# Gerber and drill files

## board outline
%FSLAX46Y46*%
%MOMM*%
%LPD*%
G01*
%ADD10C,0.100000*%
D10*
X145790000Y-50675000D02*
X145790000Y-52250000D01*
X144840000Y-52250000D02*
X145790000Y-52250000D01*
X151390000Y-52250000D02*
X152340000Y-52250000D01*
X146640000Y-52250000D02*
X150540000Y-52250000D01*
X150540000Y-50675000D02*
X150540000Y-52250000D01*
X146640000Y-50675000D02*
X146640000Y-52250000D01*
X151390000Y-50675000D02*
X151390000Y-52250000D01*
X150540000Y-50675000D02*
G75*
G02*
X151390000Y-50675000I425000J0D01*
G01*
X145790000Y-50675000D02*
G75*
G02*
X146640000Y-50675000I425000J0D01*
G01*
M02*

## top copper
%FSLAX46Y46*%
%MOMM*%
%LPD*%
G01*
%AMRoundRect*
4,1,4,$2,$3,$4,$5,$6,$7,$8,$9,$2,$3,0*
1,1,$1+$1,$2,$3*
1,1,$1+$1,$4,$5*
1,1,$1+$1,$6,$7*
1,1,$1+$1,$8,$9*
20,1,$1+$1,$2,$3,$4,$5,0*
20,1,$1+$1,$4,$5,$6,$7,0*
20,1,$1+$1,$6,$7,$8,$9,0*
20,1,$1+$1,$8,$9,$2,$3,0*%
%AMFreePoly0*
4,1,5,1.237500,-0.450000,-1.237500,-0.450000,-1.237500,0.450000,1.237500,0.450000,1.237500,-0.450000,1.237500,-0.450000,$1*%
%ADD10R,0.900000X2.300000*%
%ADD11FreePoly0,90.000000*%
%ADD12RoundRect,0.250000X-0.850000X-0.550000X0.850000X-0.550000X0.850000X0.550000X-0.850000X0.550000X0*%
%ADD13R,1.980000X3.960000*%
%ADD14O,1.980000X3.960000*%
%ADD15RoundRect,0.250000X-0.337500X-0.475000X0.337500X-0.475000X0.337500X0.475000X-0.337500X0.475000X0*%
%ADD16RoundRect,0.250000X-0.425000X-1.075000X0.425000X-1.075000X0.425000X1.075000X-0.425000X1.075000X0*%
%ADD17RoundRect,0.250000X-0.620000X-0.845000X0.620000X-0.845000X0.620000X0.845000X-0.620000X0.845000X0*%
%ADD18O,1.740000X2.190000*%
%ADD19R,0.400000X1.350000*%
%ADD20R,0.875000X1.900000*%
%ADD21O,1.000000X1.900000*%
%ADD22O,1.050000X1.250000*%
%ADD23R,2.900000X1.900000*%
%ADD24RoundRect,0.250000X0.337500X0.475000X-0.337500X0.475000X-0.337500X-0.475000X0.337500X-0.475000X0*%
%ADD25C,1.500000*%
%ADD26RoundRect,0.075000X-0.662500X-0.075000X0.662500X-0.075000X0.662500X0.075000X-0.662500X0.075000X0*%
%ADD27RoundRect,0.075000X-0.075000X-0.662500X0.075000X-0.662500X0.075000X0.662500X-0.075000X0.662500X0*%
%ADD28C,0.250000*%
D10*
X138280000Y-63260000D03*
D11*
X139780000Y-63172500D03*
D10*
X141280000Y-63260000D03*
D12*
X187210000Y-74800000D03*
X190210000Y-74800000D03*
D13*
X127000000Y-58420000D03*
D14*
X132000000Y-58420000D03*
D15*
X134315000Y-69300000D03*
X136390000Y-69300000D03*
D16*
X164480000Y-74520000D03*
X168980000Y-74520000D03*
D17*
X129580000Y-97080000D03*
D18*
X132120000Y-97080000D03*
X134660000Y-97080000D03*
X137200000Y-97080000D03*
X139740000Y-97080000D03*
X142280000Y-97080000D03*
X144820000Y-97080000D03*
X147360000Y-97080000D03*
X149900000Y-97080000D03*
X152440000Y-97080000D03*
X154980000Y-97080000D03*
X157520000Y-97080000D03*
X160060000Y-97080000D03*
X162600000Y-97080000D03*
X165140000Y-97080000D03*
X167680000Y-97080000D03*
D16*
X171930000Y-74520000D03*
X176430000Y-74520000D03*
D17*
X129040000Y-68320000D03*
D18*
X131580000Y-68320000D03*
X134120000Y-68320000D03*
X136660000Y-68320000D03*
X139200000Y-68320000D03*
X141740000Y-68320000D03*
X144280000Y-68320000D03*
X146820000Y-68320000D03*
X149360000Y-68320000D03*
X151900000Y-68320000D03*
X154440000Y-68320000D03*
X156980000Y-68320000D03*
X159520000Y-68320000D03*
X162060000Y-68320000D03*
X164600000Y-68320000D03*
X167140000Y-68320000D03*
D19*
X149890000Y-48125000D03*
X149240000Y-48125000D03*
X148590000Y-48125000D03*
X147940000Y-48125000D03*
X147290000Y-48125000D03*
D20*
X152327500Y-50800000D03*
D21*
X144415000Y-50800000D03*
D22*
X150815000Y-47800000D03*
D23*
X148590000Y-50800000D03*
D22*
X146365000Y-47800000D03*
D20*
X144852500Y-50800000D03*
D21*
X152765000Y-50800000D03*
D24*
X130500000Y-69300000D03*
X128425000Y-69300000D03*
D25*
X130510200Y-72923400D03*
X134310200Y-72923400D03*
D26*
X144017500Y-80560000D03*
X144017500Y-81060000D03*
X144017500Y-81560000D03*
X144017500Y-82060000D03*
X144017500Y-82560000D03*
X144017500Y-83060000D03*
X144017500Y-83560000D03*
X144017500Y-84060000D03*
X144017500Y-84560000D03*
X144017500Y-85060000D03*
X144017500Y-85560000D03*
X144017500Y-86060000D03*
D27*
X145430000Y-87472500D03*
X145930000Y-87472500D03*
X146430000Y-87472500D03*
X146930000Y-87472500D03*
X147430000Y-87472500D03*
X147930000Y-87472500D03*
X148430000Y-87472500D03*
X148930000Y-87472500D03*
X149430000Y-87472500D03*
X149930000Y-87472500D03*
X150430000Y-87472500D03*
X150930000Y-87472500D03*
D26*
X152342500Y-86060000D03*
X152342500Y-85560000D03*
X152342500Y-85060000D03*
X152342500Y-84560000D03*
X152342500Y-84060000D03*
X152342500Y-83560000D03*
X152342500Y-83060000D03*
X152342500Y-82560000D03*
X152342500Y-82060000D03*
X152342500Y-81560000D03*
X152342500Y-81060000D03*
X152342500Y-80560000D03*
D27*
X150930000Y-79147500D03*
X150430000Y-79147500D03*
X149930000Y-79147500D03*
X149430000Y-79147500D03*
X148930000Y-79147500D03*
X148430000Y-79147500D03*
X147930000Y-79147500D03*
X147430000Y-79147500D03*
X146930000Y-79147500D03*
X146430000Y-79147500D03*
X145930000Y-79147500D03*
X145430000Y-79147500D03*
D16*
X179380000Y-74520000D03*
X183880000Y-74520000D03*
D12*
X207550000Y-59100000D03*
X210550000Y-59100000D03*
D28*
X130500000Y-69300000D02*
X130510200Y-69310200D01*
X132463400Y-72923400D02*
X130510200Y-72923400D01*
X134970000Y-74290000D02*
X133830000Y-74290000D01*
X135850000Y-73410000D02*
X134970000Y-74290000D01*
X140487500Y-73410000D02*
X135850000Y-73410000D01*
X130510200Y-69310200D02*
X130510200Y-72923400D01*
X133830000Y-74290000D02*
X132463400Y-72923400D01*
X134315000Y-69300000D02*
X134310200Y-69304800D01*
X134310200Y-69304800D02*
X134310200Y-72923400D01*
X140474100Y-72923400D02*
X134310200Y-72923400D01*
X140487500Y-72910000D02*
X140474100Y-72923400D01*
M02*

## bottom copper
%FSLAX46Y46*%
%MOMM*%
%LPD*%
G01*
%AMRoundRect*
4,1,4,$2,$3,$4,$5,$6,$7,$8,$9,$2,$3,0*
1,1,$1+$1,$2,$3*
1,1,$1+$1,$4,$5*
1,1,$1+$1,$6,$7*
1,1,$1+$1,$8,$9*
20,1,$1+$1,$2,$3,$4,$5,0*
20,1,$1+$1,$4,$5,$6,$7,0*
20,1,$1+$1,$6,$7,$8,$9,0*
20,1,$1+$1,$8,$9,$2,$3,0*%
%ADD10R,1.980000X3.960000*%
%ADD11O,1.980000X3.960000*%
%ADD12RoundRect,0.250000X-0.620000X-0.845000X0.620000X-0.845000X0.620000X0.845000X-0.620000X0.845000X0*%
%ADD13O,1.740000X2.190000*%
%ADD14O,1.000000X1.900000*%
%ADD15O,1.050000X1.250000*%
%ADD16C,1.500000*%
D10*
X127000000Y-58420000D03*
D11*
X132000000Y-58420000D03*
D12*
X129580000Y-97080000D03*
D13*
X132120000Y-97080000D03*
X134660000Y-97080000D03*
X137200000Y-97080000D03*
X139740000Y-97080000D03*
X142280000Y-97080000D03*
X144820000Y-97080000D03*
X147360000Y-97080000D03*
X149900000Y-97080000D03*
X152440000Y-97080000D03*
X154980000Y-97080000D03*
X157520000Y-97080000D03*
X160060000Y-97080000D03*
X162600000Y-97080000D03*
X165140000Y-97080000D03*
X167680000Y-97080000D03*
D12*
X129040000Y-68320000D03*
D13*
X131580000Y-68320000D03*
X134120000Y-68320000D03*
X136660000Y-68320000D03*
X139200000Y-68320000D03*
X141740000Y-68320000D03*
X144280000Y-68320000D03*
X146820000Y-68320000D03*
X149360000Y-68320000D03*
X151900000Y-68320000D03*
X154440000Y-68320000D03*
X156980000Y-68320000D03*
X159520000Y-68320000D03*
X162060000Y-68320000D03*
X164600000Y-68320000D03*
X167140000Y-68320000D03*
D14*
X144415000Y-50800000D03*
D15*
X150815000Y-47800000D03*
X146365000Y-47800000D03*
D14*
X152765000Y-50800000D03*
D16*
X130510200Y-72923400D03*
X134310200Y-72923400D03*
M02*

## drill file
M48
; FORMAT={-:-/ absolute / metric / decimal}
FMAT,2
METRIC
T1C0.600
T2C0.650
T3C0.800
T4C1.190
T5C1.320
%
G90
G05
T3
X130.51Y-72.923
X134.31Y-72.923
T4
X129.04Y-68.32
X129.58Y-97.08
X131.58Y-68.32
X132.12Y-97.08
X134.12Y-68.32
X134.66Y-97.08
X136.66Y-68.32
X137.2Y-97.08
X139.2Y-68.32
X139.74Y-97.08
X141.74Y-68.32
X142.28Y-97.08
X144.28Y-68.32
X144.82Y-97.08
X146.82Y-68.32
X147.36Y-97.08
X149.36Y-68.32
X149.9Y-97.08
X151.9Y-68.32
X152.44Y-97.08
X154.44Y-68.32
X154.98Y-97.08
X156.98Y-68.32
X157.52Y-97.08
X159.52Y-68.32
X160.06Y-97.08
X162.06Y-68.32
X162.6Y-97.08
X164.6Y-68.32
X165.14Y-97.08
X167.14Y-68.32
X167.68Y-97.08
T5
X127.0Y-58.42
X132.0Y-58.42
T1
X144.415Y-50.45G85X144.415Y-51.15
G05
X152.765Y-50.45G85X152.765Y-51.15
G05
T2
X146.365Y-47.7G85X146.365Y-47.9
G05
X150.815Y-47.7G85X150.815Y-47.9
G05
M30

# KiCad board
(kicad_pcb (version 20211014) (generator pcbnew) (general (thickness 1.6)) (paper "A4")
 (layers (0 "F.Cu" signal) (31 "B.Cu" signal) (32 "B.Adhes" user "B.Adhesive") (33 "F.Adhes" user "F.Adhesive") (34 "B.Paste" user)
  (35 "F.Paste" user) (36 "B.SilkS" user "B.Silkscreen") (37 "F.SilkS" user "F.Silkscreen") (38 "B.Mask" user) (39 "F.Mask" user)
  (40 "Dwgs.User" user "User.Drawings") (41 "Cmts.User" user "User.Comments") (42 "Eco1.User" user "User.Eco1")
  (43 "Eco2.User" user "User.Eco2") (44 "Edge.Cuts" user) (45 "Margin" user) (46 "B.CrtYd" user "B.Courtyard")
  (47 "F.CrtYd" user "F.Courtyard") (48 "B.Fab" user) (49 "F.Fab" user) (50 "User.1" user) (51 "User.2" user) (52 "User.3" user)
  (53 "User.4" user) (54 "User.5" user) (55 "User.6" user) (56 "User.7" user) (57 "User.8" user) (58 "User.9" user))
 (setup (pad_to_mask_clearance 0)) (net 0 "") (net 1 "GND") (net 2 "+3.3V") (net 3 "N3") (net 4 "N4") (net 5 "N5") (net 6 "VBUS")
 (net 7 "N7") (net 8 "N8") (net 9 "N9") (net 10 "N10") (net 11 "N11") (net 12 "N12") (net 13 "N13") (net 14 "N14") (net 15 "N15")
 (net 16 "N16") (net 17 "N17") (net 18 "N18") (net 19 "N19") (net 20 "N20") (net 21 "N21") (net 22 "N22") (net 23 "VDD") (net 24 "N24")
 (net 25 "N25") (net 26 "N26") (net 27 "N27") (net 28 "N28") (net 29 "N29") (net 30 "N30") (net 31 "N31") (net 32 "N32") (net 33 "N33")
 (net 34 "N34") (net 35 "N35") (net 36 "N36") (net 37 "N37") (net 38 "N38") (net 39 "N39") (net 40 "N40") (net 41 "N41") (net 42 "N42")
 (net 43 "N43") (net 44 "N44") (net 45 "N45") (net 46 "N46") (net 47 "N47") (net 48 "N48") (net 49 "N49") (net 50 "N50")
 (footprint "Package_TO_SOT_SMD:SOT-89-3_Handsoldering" (layer "F.Cu") (at 139.78 61.11 90)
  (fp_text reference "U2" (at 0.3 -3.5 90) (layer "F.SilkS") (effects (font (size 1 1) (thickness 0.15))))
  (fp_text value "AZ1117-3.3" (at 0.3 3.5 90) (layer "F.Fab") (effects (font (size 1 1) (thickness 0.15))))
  (pad "1" smd rect (at -2.15 -1.5 90) (size 2.3 0.9) (layers "F.Cu" "F.Paste" "F.Mask") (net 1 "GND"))
  (pad "2" smd custom (at -2.0625 0 90) (size 2.475 0.9) (layers "F.Cu" "F.Paste" "F.Mask") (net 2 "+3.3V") (zone_connect 2)
   (options (clearance outline) (anchor rect)) (primitives))
  (pad "3" smd rect (at -2.15 1.5 90) (size 2.3 0.9) (layers "F.Cu" "F.Paste" "F.Mask") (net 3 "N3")))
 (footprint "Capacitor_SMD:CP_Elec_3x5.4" (layer "F.Cu") (at 188.71 74.8)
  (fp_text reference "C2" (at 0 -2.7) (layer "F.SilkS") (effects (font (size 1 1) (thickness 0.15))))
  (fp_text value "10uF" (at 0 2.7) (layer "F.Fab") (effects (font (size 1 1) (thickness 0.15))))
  (pad "1" smd roundrect (at -1.5 0) (size 2.2 1.6) (layers "F.Cu" "F.Paste" "F.Mask") (roundrect_rratio 0.15625) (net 2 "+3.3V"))
  (pad "2" smd roundrect (at 1.5 0) (size 2.2 1.6) (layers "F.Cu" "F.Paste" "F.Mask") (roundrect_rratio 0.15625) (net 1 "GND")))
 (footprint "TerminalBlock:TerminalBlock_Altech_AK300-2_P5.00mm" (layer "F.Cu") (at 127 58.42)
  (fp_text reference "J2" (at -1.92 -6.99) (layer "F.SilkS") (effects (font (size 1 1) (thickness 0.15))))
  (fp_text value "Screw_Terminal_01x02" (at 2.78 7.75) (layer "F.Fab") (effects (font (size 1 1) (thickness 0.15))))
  (pad "1" thru_hole rect (at 0 0) (size 1.98 3.96) (drill 1.32) (layers *.Cu *.Mask) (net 1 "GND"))
  (pad "2" thru_hole oval (at 5 0) (size 1.98 3.96) (drill 1.32) (layers *.Cu *.Mask) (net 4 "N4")))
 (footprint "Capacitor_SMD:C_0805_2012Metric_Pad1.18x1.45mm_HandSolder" (layer "F.Cu") (at 135.3525 69.3)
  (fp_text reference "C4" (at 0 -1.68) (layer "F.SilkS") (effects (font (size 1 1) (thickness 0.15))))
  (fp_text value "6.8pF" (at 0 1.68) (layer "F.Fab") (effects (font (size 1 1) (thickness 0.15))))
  (pad "1" smd roundrect (at -1.0375 0) (size 1.175 1.45) (layers "F.Cu" "F.Paste" "F.Mask") (roundrect_rratio 0.212766) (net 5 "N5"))
  (pad "2" smd roundrect (at 1.0375 0) (size 1.175 1.45) (layers "F.Cu" "F.Paste" "F.Mask") (roundrect_rratio 0.212766) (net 1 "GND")))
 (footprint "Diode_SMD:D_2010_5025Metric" (layer "F.Cu") (at 166.73 74.52)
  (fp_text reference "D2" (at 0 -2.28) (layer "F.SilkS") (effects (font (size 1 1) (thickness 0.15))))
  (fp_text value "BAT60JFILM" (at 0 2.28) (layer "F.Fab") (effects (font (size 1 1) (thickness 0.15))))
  (pad "1" smd roundrect (at -2.25 0) (size 1.35 2.65) (layers "F.Cu" "F.Paste" "F.Mask") (roundrect_rratio 0.185185) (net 3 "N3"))
  (pad "2" smd roundrect (at 2.25 0) (size 1.35 2.65) (layers "F.Cu" "F.Paste" "F.Mask") (roundrect_rratio 0.185185) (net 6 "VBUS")))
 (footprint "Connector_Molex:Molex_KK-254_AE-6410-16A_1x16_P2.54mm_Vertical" (layer "F.Cu") (at 129.58 97.08)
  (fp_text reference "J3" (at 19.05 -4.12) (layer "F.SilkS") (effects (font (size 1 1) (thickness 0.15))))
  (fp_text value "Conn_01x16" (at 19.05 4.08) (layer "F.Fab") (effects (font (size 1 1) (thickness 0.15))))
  (pad "1" thru_hole roundrect (at 0 0) (size 1.74 2.19) (drill 1.19) (layers *.Cu *.Mask) (roundrect_rratio 0.143678) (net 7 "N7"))
  (pad "2" thru_hole oval (at 2.54 0) (size 1.74 2.19) (drill 1.19) (layers *.Cu *.Mask) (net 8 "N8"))
  (pad "3" thru_hole oval (at 5.08 0) (size 1.74 2.19) (drill 1.19) (layers *.Cu *.Mask) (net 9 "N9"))
  (pad "4" thru_hole oval (at 7.62 0) (size 1.74 2.19) (drill 1.19) (layers *.Cu *.Mask) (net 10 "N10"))
  (pad "5" thru_hole oval (at 10.16 0) (size 1.74 2.19) (drill 1.19) (layers *.Cu *.Mask) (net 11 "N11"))
  (pad "6" thru_hole oval (at 12.7 0) (size 1.74 2.19) (drill 1.19) (layers *.Cu *.Mask) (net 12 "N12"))
  (pad "7" thru_hole oval (at 15.24 0) (size 1.74 2.19) (drill 1.19) (layers *.Cu *.Mask) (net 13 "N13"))
  (pad "8" thru_hole oval (at 17.78 0) (size 1.74 2.19) (drill 1.19) (layers *.Cu *.Mask) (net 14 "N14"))
  (pad "9" thru_hole oval (at 20.32 0) (size 1.74 2.19) (drill 1.19) (layers *.Cu *.Mask) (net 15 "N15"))
  (pad "10" thru_hole oval (at 22.86 0) (size 1.74 2.19) (drill 1.19) (layers *.Cu *.Mask) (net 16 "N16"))
  (pad "11" thru_hole oval (at 25.4 0) (size 1.74 2.19) (drill 1.19) (layers *.Cu *.Mask) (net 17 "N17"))
  (pad "12" thru_hole oval (at 27.94 0) (size 1.74 2.19) (drill 1.19) (layers *.Cu *.Mask) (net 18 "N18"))
  (pad "13" thru_hole oval (at 30.48 0) (size 1.74 2.19) (drill 1.19) (layers *.Cu *.Mask) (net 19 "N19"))
  (pad "14" thru_hole oval (at 33.02 0) (size 1.74 2.19) (drill 1.19) (layers *.Cu *.Mask) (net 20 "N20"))
  (pad "15" thru_hole oval (at 35.56 0) (size 1.74 2.19) (drill 1.19) (layers *.Cu *.Mask) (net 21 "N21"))
  (pad "16" thru_hole oval (at 38.1 0) (size 1.74 2.19) (drill 1.19) (layers *.Cu *.Mask) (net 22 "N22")))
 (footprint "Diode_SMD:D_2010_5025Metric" (layer "F.Cu") (at 174.18 74.52)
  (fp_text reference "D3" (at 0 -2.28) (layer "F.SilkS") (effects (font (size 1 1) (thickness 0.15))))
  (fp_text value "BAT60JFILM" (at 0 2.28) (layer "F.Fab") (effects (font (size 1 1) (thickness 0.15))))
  (pad "1" smd roundrect (at -2.25 0) (size 1.35 2.65) (layers "F.Cu" "F.Paste" "F.Mask") (roundrect_rratio 0.185185) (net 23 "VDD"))
  (pad "2" smd roundrect (at 2.25 0) (size 1.35 2.65) (layers "F.Cu" "F.Paste" "F.Mask") (roundrect_rratio 0.185185) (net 2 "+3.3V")))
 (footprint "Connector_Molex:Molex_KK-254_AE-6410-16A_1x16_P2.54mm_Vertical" (layer "F.Cu") (at 129.04 68.32)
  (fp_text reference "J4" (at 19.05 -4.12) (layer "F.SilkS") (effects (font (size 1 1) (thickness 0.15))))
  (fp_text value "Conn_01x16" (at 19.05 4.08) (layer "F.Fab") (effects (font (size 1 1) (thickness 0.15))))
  (pad "1" thru_hole roundrect (at 0 0) (size 1.74 2.19) (drill 1.19) (layers *.Cu *.Mask) (roundrect_rratio 0.143678) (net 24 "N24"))
  (pad "2" thru_hole oval (at 2.54 0) (size 1.74 2.19) (drill 1.19) (layers *.Cu *.Mask) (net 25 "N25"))
  (pad "3" thru_hole oval (at 5.08 0) (size 1.74 2.19) (drill 1.19) (layers *.Cu *.Mask) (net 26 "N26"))
  (pad "4" thru_hole oval (at 7.62 0) (size 1.74 2.19) (drill 1.19) (layers *.Cu *.Mask) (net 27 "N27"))
  (pad "5" thru_hole oval (at 10.16 0) (size 1.74 2.19) (drill 1.19) (layers *.Cu *.Mask) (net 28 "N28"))
  (pad "6" thru_hole oval (at 12.7 0) (size 1.74 2.19) (drill 1.19) (layers *.Cu *.Mask) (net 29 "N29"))
  (pad "7" thru_hole oval (at 15.24 0) (size 1.74 2.19) (drill 1.19) (layers *.Cu *.Mask) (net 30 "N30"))
  (pad "8" thru_hole oval (at 17.78 0) (size 1.74 2.19) (drill 1.19) (layers *.Cu *.Mask) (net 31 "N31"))
  (pad "9" thru_hole oval (at 20.32 0) (size 1.74 2.19) (drill 1.19) (layers *.Cu *.Mask) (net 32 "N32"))
  (pad "10" thru_hole oval (at 22.86 0) (size 1.74 2.19) (drill 1.19) (layers *.Cu *.Mask) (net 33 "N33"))
  (pad "11" thru_hole oval (at 25.4 0) (size 1.74 2.19) (drill 1.19) (layers *.Cu *.Mask) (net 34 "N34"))
  (pad "12" thru_hole oval (at 27.94 0) (size 1.74 2.19) (drill 1.19) (layers *.Cu *.Mask) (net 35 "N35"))
  (pad "13" thru_hole oval (at 30.48 0) (size 1.74 2.19) (drill 1.19) (layers *.Cu *.Mask) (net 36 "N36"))
  (pad "14" thru_hole oval (at 33.02 0) (size 1.74 2.19) (drill 1.19) (layers *.Cu *.Mask) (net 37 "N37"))
  (pad "15" thru_hole oval (at 35.56 0) (size 1.74 2.19) (drill 1.19) (layers *.Cu *.Mask) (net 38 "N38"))
  (pad "16" thru_hole oval (at 38.1 0) (size 1.74 2.19) (drill 1.19) (layers *.Cu *.Mask) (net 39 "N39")))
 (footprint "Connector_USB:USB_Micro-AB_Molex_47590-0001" (layer "F.Cu") (at 148.59 50.8)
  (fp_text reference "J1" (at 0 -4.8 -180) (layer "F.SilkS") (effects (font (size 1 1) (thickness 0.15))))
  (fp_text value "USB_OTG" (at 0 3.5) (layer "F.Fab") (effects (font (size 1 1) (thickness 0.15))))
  (fp_line (start -2.8 -0.125) (end -2.8 1.45) (layer "Edge.Cuts") (width 0.1))
  (fp_line (start -3.75 1.45) (end -2.8 1.45) (layer "Edge.Cuts") (width 0.1))
  (fp_line (start 2.8 1.45) (end 3.75 1.45) (layer "Edge.Cuts") (width 0.1))
  (fp_line (start -1.95 1.45) (end 1.95 1.45) (layer "Edge.Cuts") (width 0.1))
  (fp_line (start 1.95 -0.125) (end 1.95 1.45) (layer "Edge.Cuts") (width 0.1))
  (fp_line (start -1.95 -0.125) (end -1.95 1.45) (layer "Edge.Cuts") (width 0.1))
  (fp_line (start 2.8 -0.125) (end 2.8 1.45) (layer "Edge.Cuts") (width 0.1))
  (fp_arc (start 1.95 -0.125) (mid 2.375 -0.55) (end 2.8 -0.125) (layer "Edge.Cuts") (width 0.1))
  (fp_arc (start -2.8 -0.125) (mid -2.375 -0.55) (end -1.95 -0.125) (layer "Edge.Cuts") (width 0.1))
  (pad "" smd rect (at 3.5 0) (size 0.3 0.85) (layers "F.Paste"))
  (pad "" smd rect (at -3.5 0) (size 0.3 0.85) (layers "F.Paste"))
  (pad "1" smd rect (at 1.3 -2.675) (size 0.4 1.35) (layers "F.Cu" "F.Paste" "F.Mask") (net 6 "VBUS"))
  (pad "2" smd rect (at 0.65 -2.675) (size 0.4 1.35) (layers "F.Cu" "F.Paste" "F.Mask") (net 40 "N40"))
  (pad "3" smd rect (at 0 -2.675) (size 0.4 1.35) (layers "F.Cu" "F.Paste" "F.Mask") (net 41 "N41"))
  (pad "4" smd rect (at -0.65 -2.675) (size 0.4 1.35) (layers "F.Cu" "F.Paste" "F.Mask") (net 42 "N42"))
  (pad "5" smd rect (at -1.3 -2.675) (size 0.4 1.35) (layers "F.Cu" "F.Paste" "F.Mask") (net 1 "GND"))
  (pad "6" smd rect (at 3.7375 0) (size 0.875 1.9) (layers "F.Cu" "F.Mask") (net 1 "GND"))
  (pad "6" thru_hole oval (at -4.175 0) (size 1 1.9) (drill oval 0.6 1.3) (layers *.Cu *.Mask) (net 1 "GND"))
  (pad "6" thru_hole oval (at 2.225 -3) (size 1.05 1.25) (drill oval 0.65 0.85) (layers *.Cu *.Mask) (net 1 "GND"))
  (pad "6" smd rect (at 0 0) (size 2.9 1.9) (layers "F.Cu" "F.Paste" "F.Mask") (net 1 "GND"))
  (pad "6" thru_hole oval (at -2.225 -3) (size 1.05 1.25) (drill oval 0.65 0.85) (layers *.Cu *.Mask) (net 1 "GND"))
  (pad "6" smd rect (at -3.7375 0) (size 0.875 1.9) (layers "F.Cu" "F.Mask") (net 1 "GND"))
  (pad "6" thru_hole oval (at 4.175 0) (size 1 1.9) (drill oval 0.6 1.3) (layers *.Cu *.Mask) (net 1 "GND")))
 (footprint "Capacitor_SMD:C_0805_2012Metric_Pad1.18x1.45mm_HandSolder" (layer "F.Cu") (at 129.4625 69.3 180)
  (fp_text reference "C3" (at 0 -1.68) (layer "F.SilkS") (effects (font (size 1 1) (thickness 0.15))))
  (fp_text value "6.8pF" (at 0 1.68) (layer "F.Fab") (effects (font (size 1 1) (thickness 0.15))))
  (pad "1" smd roundrect (at -1.0375 0 180) (size 1.175 1.45) (layers "F.Cu" "F.Paste" "F.Mask") (roundrect_rratio 0.212766) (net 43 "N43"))
  (pad "2" smd roundrect (at 1.0375 0 180) (size 1.175 1.45) (layers "F.Cu" "F.Paste" "F.Mask") (roundrect_rratio 0.212766) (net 1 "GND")))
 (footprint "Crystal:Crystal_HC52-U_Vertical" (layer "F.Cu") (at 130.5102 72.9234)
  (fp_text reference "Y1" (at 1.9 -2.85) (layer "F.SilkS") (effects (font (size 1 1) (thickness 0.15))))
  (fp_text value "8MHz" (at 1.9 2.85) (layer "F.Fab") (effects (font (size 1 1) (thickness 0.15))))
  (pad "1" thru_hole circle (at 0 0) (size 1.5 1.5) (drill 0.8) (layers *.Cu *.Mask) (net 43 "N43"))
  (pad "2" thru_hole circle (at 3.8 0) (size 1.5 1.5) (drill 0.8) (layers *.Cu *.Mask) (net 5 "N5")))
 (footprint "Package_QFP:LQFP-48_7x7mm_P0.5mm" (layer "F.Cu") (at 148.18 83.31)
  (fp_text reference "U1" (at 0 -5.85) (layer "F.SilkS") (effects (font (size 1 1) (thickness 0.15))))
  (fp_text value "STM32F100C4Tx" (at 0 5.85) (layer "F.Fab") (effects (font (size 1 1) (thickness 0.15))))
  (pad "1" smd roundrect (at -4.1625 -2.75) (size 1.475 0.3) (layers "F.Cu" "F.Paste" "F.Mask") (roundrect_rratio 0.25) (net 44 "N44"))
  (pad "2" smd roundrect (at -4.1625 -2.25) (size 1.475 0.3) (layers "F.Cu" "F.Paste" "F.Mask") (roundrect_rratio 0.25) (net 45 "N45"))
  (pad "3" smd roundrect (at -4.1625 -1.75) (size 1.475 0.3) (layers "F.Cu" "F.Paste" "F.Mask") (roundrect_rratio 0.25) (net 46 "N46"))
  (pad "4" smd roundrect (at -4.1625 -1.25) (size 1.475 0.3) (layers "F.Cu" "F.Paste" "F.Mask") (roundrect_rratio 0.25) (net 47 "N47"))
  (pad "5" smd roundrect (at -4.1625 -0.75) (size 1.475 0.3) (layers "F.Cu" "F.Paste" "F.Mask") (roundrect_rratio 0.25) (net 5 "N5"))
  (pad "6" smd roundrect (at -4.1625 -0.25) (size 1.475 0.3) (layers "F.Cu" "F.Paste" "F.Mask") (roundrect_rratio 0.25) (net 43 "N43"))
  (pad "7" smd roundrect (at -4.1625 0.25) (size 1.475 0.3) (layers "F.Cu" "F.Paste" "F.Mask") (roundrect_rratio 0.25) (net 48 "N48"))
  (pad "8" smd roundrect (at -4.1625 0.75) (size 1.475 0.3) (layers "F.Cu" "F.Paste" "F.Mask") (roundrect_rratio 0.25) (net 1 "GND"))
  (pad "9" smd roundrect (at -4.1625 1.25) (size 1.475 0.3) (layers "F.Cu" "F.Paste" "F.Mask") (roundrect_rratio 0.25) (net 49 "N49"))
  (pad "10" smd roundrect (at -4.1625 1.75) (size 1.475 0.3) (layers "F.Cu" "F.Paste" "F.Mask") (roundrect_rratio 0.25) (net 7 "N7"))
  (pad "11" smd roundrect (at -4.1625 2.25) (size 1.475 0.3) (layers "F.Cu" "F.Paste" "F.Mask") (roundrect_rratio 0.25) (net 8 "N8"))
  (pad "12" smd roundrect (at -4.1625 2.75) (size 1.475 0.3) (layers "F.Cu" "F.Paste" "F.Mask") (roundrect_rratio 0.25) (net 9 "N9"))
  (pad "13" smd roundrect (at -2.75 4.1625) (size 0.3 1.475) (layers "F.Cu" "F.Paste" "F.Mask") (roundrect_rratio 0.25) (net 10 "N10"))
  (pad "14" smd roundrect (at -2.25 4.1625) (size 0.3 1.475) (layers "F.Cu" "F.Paste" "F.Mask") (roundrect_rratio 0.25) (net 11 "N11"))
  (pad "15" smd roundrect (at -1.75 4.1625) (size 0.3 1.475) (layers "F.Cu" "F.Paste" "F.Mask") (roundrect_rratio 0.25) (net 12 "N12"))
  (pad "16" smd roundrect (at -1.25 4.1625) (size 0.3 1.475) (layers "F.Cu" "F.Paste" "F.Mask") (roundrect_rratio 0.25) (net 13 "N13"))
  (pad "17" smd roundrect (at -0.75 4.1625) (size 0.3 1.475) (layers "F.Cu" "F.Paste" "F.Mask") (roundrect_rratio 0.25) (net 14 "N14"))
  (pad "18" smd roundrect (at -0.25 4.1625) (size 0.3 1.475) (layers "F.Cu" "F.Paste" "F.Mask") (roundrect_rratio 0.25) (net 24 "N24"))
  (pad "19" smd roundrect (at 0.25 4.1625) (size 0.3 1.475) (layers "F.Cu" "F.Paste" "F.Mask") (roundrect_rratio 0.25) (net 25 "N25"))
  (pad "20" smd roundrect (at 0.75 4.1625) (size 0.3 1.475) (layers "F.Cu" "F.Paste" "F.Mask") (roundrect_rratio 0.25) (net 26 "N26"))
  (pad "21" smd roundrect (at 1.25 4.1625) (size 0.3 1.475) (layers "F.Cu" "F.Paste" "F.Mask") (roundrect_rratio 0.25) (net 34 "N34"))
  (pad "22" smd roundrect (at 1.75 4.1625) (size 0.3 1.475) (layers "F.Cu" "F.Paste" "F.Mask") (roundrect_rratio 0.25) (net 35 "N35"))
  (pad "23" smd roundrect (at 2.25 4.1625) (size 0.3 1.475) (layers "F.Cu" "F.Paste" "F.Mask") (roundrect_rratio 0.25) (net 1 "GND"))
  (pad "24" smd roundrect (at 2.75 4.1625) (size 0.3 1.475) (layers "F.Cu" "F.Paste" "F.Mask") (roundrect_rratio 0.25) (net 23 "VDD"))
  (pad "25" smd roundrect (at 4.1625 2.75) (size 1.475 0.3) (layers "F.Cu" "F.Paste" "F.Mask") (roundrect_rratio 0.25) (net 36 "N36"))
  (pad "26" smd roundrect (at 4.1625 2.25) (size 1.475 0.3) (layers "F.Cu" "F.Paste" "F.Mask") (roundrect_rratio 0.25) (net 37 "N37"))
  (pad "27" smd roundrect (at 4.1625 1.75) (size 1.475 0.3) (layers "F.Cu" "F.Paste" "F.Mask") (roundrect_rratio 0.25) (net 38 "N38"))
  (pad "28" smd roundrect (at 4.1625 1.25) (size 1.475 0.3) (layers "F.Cu" "F.Paste" "F.Mask") (roundrect_rratio 0.25) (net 39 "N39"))
  (pad "29" smd roundrect (at 4.1625 0.75) (size 1.475 0.3) (layers "F.Cu" "F.Paste" "F.Mask") (roundrect_rratio 0.25) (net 15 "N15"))
  (pad "30" smd roundrect (at 4.1625 0.25) (size 1.475 0.3) (layers "F.Cu" "F.Paste" "F.Mask") (roundrect_rratio 0.25) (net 16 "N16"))
  (pad "31" smd roundrect (at 4.1625 -0.25) (size 1.475 0.3) (layers "F.Cu" "F.Paste" "F.Mask") (roundrect_rratio 0.25) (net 17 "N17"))
  (pad "32" smd roundrect (at 4.1625 -0.75) (size 1.475 0.3) (layers "F.Cu" "F.Paste" "F.Mask") (roundrect_rratio 0.25) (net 18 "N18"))
  (pad "33" smd roundrect (at 4.1625 -1.25) (size 1.475 0.3) (layers "F.Cu" "F.Paste" "F.Mask") (roundrect_rratio 0.25) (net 19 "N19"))
  (pad "34" smd roundrect (at 4.1625 -1.75) (size 1.475 0.3) (layers "F.Cu" "F.Paste" "F.Mask") (roundrect_rratio 0.25) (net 20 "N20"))
  (pad "35" smd roundrect (at 4.1625 -2.25) (size 1.475 0.3) (layers "F.Cu" "F.Paste" "F.Mask") (roundrect_rratio 0.25) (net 1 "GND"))
  (pad "36" smd roundrect (at 4.1625 -2.75) (size 1.475 0.3) (layers "F.Cu" "F.Paste" "F.Mask") (roundrect_rratio 0.25) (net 23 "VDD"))
  (pad "37" smd roundrect (at 2.75 -4.1625) (size 0.3 1.475) (layers "F.Cu" "F.Paste" "F.Mask") (roundrect_rratio 0.25) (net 21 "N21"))
  (pad "38" smd roundrect (at 2.25 -4.1625) (size 0.3 1.475) (layers "F.Cu" "F.Paste" "F.Mask") (roundrect_rratio 0.25) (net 22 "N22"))
  (pad "39" smd roundrect (at 1.75 -4.1625) (size 0.3 1.475) (layers "F.Cu" "F.Paste" "F.Mask") (roundrect_rratio 0.25) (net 27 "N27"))
  (pad "40" smd roundrect (at 1.25 -4.1625) (size 0.3 1.475) (layers "F.Cu" "F.Paste" "F.Mask") (roundrect_rratio 0.25) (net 28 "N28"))
  (pad "41" smd roundrect (at 0.75 -4.1625) (size 0.3 1.475) (layers "F.Cu" "F.Paste" "F.Mask") (roundrect_rratio 0.25) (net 29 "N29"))
  (pad "42" smd roundrect (at 0.25 -4.1625) (size 0.3 1.475) (layers "F.Cu" "F.Paste" "F.Mask") (roundrect_rratio 0.25) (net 30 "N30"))
  (pad "43" smd roundrect (at -0.25 -4.1625) (size 0.3 1.475) (layers "F.Cu" "F.Paste" "F.Mask") (roundrect_rratio 0.25) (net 31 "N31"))
  (pad "44" smd roundrect (at -0.75 -4.1625) (size 0.3 1.475) (layers "F.Cu" "F.Paste" "F.Mask") (roundrect_rratio 0.25) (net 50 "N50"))
  (pad "45" smd roundrect (at -1.25 -4.1625) (size 0.3 1.475) (layers "F.Cu" "F.Paste" "F.Mask") (roundrect_rratio 0.25) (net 32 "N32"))
  (pad "46" smd roundrect (at -1.75 -4.1625) (size 0.3 1.475) (layers "F.Cu" "F.Paste" "F.Mask") (roundrect_rratio 0.25) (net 33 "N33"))
  (pad "47" smd roundrect (at -2.25 -4.1625) (size 0.3 1.475) (layers "F.Cu" "F.Paste" "F.Mask") (roundrect_rratio 0.25) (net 1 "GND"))
  (pad "48" smd roundrect (at -2.75 -4.1625) (size 0.3 1.475) (layers "F.Cu" "F.Paste" "F.Mask") (roundrect_rratio 0.25) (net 23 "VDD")))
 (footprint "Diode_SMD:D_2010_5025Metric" (layer "F.Cu") (at 181.63 74.52)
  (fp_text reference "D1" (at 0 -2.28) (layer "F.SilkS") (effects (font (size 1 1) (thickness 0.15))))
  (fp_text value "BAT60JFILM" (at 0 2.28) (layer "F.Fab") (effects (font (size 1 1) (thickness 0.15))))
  (pad "1" smd roundrect (at -2.25 0) (size 1.35 2.65) (layers "F.Cu" "F.Paste" "F.Mask") (roundrect_rratio 0.185185) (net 3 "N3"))
  (pad "2" smd roundrect (at 2.25 0) (size 1.35 2.65) (layers "F.Cu" "F.Paste" "F.Mask") (roundrect_rratio 0.185185) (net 4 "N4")))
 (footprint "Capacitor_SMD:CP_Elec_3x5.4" (layer "F.Cu") (at 209.05 59.1)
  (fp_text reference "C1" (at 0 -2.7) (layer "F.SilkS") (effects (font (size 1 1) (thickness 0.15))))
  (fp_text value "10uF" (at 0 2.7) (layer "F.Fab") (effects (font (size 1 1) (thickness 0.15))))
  (pad "1" smd roundrect (at -1.5 0) (size 2.2 1.6) (layers "F.Cu" "F.Paste" "F.Mask") (roundrect_rratio 0.15625) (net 3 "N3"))
  (pad "2" smd roundrect (at 1.5 0) (size 2.2 1.6) (layers "F.Cu" "F.Paste" "F.Mask") (roundrect_rratio 0.15625) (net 1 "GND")))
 (segment (start 130.5 69.3) (end 130.5102 69.3102) (width 0.25) (layer "F.Cu") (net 43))
 (segment (start 132.4634 72.9234) (end 130.5102 72.9234) (width 0.25) (layer "F.Cu") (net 43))
 (segment (start 134.97 74.29) (end 133.83 74.29) (width 0.25) (layer "F.Cu") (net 43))
 (segment (start 135.85 73.41) (end 134.97 74.29) (width 0.25) (layer "F.Cu") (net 43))
 (segment (start 140.4875 73.41) (end 135.85 73.41) (width 0.25) (layer "F.Cu") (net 43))
 (segment (start 130.5102 69.3102) (end 130.5102 72.9234) (width 0.25) (layer "F.Cu") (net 43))
 (segment (start 133.83 74.29) (end 132.4634 72.9234) (width 0.25) (layer "F.Cu") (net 43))
 (segment (start 134.315 69.3) (end 134.3102 69.3048) (width 0.25) (layer "F.Cu") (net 5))
 (segment (start 134.3102 69.3048) (end 134.3102 72.9234) (width 0.25) (layer "F.Cu") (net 5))
 (segment (start 140.4741 72.9234) (end 134.3102 72.9234) (width 0.25) (layer "F.Cu") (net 5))
 (segment (start 140.4875 72.91) (end 140.4741 72.9234) (width 0.25) (layer "F.Cu") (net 5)))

